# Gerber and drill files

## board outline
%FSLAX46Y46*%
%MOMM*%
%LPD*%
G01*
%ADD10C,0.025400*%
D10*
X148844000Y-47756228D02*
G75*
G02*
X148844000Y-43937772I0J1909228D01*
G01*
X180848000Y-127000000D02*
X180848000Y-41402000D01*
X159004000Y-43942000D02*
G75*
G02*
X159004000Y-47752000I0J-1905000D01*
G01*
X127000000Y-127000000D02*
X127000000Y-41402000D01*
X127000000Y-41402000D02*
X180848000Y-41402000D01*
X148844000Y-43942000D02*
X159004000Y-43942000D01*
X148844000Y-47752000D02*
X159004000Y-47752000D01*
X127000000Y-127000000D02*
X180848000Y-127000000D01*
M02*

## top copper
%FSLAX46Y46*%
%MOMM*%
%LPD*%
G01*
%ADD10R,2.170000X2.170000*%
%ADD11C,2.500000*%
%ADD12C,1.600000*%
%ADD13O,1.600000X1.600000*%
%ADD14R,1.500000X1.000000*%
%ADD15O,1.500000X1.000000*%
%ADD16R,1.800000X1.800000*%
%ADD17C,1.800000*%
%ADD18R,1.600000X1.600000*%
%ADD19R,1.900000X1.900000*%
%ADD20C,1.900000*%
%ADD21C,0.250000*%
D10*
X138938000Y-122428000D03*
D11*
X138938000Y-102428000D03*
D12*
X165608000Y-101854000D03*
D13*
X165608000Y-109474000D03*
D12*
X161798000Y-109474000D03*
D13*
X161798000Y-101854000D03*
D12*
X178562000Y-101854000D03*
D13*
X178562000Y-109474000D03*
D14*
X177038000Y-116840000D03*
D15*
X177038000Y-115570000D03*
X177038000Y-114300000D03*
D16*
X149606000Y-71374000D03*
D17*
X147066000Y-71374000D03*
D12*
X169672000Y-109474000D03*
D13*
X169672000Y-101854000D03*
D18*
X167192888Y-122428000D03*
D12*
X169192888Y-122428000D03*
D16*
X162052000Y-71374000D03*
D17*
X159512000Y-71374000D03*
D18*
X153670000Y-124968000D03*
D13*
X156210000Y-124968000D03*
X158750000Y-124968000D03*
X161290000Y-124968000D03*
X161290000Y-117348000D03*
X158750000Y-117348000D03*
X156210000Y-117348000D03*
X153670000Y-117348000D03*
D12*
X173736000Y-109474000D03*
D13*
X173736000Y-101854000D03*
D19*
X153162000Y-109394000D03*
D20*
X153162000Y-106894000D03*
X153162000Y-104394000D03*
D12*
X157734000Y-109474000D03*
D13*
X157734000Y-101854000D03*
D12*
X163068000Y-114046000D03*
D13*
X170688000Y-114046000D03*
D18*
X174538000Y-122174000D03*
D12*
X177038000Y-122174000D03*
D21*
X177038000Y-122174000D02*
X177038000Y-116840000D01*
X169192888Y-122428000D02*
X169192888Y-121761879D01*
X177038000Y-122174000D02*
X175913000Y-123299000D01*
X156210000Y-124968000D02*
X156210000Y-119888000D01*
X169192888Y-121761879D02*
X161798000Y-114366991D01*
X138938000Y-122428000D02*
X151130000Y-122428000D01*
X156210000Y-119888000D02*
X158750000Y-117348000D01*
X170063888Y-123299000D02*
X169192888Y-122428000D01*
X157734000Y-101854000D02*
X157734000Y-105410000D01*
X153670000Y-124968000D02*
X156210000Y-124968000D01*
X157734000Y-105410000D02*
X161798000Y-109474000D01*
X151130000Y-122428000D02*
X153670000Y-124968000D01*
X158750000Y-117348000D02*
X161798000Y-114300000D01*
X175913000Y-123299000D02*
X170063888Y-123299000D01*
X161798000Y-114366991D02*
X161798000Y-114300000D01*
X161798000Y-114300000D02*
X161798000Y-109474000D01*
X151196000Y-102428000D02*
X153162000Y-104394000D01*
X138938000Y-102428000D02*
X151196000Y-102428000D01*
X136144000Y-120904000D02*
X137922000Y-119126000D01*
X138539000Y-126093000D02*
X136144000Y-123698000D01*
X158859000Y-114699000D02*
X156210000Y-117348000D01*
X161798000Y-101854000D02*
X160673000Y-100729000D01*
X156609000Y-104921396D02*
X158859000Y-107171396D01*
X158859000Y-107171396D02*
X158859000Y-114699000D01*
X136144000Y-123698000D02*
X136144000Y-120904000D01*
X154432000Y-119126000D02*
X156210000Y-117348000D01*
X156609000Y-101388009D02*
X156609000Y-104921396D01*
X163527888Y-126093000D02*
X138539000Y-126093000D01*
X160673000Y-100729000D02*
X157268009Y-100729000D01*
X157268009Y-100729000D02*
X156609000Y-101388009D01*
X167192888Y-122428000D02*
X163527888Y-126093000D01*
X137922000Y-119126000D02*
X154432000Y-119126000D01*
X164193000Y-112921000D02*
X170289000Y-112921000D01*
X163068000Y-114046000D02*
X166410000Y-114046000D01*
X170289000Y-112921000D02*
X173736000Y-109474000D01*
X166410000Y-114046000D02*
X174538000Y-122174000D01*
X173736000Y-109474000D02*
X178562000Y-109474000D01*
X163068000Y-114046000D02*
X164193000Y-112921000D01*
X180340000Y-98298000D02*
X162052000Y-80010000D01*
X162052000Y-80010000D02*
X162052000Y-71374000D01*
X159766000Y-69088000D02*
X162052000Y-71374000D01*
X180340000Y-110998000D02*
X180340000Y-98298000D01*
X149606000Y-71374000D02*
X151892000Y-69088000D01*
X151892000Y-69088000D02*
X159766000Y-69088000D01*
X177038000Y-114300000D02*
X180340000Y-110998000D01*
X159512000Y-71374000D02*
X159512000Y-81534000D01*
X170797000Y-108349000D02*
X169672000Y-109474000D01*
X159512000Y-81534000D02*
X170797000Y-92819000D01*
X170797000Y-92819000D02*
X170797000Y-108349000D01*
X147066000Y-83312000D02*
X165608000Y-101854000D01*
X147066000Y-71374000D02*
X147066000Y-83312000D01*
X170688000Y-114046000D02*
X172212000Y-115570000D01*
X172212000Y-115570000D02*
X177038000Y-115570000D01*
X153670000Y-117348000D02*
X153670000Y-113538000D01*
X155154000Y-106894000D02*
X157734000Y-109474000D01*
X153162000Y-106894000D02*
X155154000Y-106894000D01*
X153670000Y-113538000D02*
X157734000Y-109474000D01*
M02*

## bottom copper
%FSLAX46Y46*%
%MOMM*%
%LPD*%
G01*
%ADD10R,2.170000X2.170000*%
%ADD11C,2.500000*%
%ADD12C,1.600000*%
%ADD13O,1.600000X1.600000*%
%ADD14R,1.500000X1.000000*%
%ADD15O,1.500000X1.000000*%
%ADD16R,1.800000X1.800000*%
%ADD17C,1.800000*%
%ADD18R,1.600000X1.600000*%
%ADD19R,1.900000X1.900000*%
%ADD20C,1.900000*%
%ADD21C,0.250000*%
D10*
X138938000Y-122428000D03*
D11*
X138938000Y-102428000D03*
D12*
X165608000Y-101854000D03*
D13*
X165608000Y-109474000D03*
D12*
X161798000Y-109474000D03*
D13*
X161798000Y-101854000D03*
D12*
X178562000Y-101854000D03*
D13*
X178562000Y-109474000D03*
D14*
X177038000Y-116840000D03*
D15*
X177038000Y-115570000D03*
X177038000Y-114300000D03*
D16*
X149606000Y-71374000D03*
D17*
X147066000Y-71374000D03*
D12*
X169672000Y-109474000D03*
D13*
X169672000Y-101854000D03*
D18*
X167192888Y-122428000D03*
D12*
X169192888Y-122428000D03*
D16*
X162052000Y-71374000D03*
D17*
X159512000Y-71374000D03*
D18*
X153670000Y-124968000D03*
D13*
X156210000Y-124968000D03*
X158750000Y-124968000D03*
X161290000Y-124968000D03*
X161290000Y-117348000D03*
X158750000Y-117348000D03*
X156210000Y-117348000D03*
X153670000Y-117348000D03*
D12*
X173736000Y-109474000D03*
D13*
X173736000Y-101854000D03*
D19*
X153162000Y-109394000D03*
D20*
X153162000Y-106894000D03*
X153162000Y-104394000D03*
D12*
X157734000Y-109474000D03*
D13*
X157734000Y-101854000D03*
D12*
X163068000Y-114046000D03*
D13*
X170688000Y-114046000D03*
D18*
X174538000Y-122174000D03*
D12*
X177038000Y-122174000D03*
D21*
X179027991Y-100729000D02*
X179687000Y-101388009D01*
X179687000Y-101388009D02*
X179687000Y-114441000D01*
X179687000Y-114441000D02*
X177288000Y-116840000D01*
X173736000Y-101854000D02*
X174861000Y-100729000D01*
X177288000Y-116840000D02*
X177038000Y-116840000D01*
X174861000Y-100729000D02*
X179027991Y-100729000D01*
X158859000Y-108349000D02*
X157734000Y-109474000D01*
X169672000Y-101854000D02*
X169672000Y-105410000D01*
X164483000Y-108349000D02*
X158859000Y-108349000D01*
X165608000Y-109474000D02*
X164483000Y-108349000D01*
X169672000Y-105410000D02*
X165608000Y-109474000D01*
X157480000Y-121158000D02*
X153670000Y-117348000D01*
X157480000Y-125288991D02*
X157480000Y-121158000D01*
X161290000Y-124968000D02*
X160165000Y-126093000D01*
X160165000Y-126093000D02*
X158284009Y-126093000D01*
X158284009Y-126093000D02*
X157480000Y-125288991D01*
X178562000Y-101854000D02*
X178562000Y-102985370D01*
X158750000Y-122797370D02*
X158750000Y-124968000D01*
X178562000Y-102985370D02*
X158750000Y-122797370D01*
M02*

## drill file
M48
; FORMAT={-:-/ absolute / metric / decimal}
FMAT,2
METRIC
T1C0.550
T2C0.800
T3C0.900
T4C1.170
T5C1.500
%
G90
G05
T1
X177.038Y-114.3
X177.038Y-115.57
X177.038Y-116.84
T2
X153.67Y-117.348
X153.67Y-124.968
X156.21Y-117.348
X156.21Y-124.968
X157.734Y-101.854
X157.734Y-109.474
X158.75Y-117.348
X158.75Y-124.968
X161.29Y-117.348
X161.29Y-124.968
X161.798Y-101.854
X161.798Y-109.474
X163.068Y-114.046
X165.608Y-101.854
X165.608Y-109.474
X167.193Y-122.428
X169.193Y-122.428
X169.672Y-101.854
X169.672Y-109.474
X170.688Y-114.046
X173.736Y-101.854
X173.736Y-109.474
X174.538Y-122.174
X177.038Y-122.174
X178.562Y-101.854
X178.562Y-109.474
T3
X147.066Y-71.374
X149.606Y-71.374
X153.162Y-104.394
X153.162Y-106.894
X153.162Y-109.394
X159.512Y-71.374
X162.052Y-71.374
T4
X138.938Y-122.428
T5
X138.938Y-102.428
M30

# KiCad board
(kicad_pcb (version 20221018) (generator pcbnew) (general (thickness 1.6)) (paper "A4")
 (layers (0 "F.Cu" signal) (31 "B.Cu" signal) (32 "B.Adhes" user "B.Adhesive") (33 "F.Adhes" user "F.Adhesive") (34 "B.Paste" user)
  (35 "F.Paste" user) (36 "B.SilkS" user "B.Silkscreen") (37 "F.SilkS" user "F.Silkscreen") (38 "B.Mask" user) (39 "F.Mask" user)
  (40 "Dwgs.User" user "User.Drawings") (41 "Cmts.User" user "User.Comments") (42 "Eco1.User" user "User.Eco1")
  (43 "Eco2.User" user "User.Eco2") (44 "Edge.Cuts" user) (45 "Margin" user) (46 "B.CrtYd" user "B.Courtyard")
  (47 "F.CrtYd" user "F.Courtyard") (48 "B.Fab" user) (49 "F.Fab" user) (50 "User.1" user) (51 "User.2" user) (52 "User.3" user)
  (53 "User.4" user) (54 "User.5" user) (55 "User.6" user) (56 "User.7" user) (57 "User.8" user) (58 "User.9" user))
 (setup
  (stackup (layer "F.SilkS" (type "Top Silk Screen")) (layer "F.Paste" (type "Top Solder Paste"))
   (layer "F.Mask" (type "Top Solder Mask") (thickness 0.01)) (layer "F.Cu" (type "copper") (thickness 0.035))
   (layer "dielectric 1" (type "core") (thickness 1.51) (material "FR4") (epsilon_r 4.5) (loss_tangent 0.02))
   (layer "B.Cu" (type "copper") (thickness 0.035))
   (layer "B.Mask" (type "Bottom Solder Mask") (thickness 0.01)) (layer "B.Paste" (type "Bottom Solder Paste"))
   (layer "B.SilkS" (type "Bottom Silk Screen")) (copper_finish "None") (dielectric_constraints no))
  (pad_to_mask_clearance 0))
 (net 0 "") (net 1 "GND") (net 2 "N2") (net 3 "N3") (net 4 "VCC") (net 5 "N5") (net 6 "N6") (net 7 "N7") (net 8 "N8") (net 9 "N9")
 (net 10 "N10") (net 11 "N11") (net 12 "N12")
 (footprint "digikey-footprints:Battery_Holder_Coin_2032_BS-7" (layer "F.Cu") (at 138.938 122.428 90)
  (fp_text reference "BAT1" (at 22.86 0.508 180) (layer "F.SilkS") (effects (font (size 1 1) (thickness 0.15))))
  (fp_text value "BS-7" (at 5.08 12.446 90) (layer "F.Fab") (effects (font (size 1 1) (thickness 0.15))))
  (pad "Neg" thru_hole rect (at 0 0 90) (size 2.17 2.17) (drill 1.17) (layers "*.Cu" "*.Mask") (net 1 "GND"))
  (pad "Pos" thru_hole circle (at 20 0 90) (size 2.5 2.5) (drill 1.5) (layers "*.Cu" "*.Mask") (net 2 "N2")))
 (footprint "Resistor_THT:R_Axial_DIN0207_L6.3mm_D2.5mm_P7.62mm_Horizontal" (layer "F.Cu") (at 165.608 101.854 -90)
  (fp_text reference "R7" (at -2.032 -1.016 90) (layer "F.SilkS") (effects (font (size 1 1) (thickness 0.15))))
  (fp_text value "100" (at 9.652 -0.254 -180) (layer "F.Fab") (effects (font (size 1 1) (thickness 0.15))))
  (pad "1" thru_hole circle (at 0 0 270) (size 1.6 1.6) (drill 0.8) (layers "*.Cu" "*.Mask") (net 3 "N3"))
  (pad "2" thru_hole oval (at 7.62 0 270) (size 1.6 1.6) (drill 0.8) (layers "*.Cu" "*.Mask") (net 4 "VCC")))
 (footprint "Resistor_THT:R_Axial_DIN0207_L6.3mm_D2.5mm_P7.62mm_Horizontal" (layer "F.Cu") (at 161.798 109.474 90)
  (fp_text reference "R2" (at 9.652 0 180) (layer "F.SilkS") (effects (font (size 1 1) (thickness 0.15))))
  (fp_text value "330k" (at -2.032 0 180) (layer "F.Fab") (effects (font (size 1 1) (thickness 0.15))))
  (pad "1" thru_hole circle (at 0 0 90) (size 1.6 1.6) (drill 0.8) (layers "*.Cu" "*.Mask") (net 1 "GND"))
  (pad "2" thru_hole oval (at 7.62 0 90) (size 1.6 1.6) (drill 0.8) (layers "*.Cu" "*.Mask") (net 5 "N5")))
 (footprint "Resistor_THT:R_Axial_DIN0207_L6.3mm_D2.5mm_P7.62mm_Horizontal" (layer "F.Cu") (at 178.562 101.854 -90)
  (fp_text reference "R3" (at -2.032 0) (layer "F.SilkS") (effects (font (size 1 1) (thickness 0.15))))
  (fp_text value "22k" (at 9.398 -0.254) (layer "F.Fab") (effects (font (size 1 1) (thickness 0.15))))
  (pad "1" thru_hole circle (at 0 0 270) (size 1.6 1.6) (drill 0.8) (layers "*.Cu" "*.Mask") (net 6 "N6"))
  (pad "2" thru_hole oval (at 7.62 0 270) (size 1.6 1.6) (drill 0.8) (layers "*.Cu" "*.Mask") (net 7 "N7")))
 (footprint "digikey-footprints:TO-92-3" (layer "F.Cu") (at 177.038 116.84 90)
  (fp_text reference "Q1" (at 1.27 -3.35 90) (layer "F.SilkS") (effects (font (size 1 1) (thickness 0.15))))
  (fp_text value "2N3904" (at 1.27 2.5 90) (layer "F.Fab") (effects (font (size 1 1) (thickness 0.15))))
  (pad "1" thru_hole rect (at 0 0 270) (size 1 1.5) (drill 0.55) (layers "*.Cu" "*.Mask") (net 1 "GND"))
  (pad "2" thru_hole oval (at 1.27 0 270) (size 1 1.5) (drill 0.55) (layers "*.Cu" "*.Mask") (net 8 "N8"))
  (pad "3" thru_hole oval (at 2.54 0 270) (size 1 1.5) (drill 0.55) (layers "*.Cu" "*.Mask") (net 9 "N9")))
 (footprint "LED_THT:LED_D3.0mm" (layer "F.Cu") (at 149.606 71.374 180)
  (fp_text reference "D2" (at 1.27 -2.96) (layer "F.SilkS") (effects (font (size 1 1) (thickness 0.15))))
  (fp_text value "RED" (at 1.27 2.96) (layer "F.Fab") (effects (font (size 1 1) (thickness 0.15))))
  (pad "1" thru_hole rect (at 0 0 180) (size 1.8 1.8) (drill 0.9) (layers "*.Cu" "*.Mask") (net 9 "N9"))
  (pad "2" thru_hole circle (at 2.54 0 180) (size 1.8 1.8) (drill 0.9) (layers "*.Cu" "*.Mask") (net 3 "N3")))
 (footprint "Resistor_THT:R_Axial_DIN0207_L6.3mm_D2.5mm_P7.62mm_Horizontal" (layer "F.Cu") (at 169.672 109.474 90)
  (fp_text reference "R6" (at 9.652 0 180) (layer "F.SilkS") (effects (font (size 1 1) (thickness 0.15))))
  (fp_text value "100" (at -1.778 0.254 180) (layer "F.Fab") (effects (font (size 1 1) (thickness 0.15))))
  (pad "1" thru_hole circle (at 0 0 90) (size 1.6 1.6) (drill 0.8) (layers "*.Cu" "*.Mask") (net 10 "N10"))
  (pad "2" thru_hole oval (at 7.62 0 90) (size 1.6 1.6) (drill 0.8) (layers "*.Cu" "*.Mask") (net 4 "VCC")))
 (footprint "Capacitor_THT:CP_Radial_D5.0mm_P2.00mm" (layer "F.Cu") (at 167.192888 122.428)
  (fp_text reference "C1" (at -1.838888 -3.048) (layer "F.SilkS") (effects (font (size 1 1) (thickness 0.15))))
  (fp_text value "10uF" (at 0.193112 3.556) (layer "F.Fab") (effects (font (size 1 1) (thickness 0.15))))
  (pad "1" thru_hole rect (at 0 0) (size 1.6 1.6) (drill 0.8) (layers "*.Cu" "*.Mask") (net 5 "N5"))
  (pad "2" thru_hole circle (at 2 0) (size 1.6 1.6) (drill 0.8) (layers "*.Cu" "*.Mask") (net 1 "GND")))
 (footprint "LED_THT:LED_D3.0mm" (layer "F.Cu") (at 162.052 71.374 180)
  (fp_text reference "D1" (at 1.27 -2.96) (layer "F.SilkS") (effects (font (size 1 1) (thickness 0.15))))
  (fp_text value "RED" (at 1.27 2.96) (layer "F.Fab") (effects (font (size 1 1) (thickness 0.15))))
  (pad "1" thru_hole rect (at 0 0 180) (size 1.8 1.8) (drill 0.9) (layers "*.Cu" "*.Mask") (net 9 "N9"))
  (pad "2" thru_hole circle (at 2.54 0 180) (size 1.8 1.8) (drill 0.9) (layers "*.Cu" "*.Mask") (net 10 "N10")))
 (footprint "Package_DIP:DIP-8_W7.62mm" (layer "F.Cu") (at 153.67 124.968 90)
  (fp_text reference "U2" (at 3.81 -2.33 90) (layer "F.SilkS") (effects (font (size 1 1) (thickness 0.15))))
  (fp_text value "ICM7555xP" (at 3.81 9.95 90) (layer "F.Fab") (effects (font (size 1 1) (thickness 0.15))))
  (pad "1" thru_hole rect (at 0 0 90) (size 1.6 1.6) (drill 0.8) (layers "*.Cu" "*.Mask") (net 1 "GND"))
  (pad "2" thru_hole oval (at 0 2.54 90) (size 1.6 1.6) (drill 0.8) (layers "*.Cu" "*.Mask") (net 1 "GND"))
  (pad "3" thru_hole oval (at 0 5.08 90) (size 1.6 1.6) (drill 0.8) (layers "*.Cu" "*.Mask") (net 6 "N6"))
  (pad "4" thru_hole oval (at 0 7.62 90) (size 1.6 1.6) (drill 0.8) (layers "*.Cu" "*.Mask") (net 4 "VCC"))
  (pad "5" thru_hole oval (at 7.62 7.62 90) (size 1.6 1.6) (drill 0.8) (layers "*.Cu" "*.Mask") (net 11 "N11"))
  (pad "6" thru_hole oval (at 7.62 5.08 90) (size 1.6 1.6) (drill 0.8) (layers "*.Cu" "*.Mask") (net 1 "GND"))
  (pad "7" thru_hole oval (at 7.62 2.54 90) (size 1.6 1.6) (drill 0.8) (layers "*.Cu" "*.Mask") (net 5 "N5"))
  (pad "8" thru_hole oval (at 7.62 0 90) (size 1.6 1.6) (drill 0.8) (layers "*.Cu" "*.Mask") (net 4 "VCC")))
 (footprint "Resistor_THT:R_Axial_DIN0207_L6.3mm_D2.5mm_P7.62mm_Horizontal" (layer "F.Cu") (at 173.736 109.474 90)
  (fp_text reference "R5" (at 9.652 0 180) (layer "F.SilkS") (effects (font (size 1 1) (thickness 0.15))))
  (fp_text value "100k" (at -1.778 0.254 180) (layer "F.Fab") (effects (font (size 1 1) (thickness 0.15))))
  (pad "1" thru_hole circle (at 0 0 90) (size 1.6 1.6) (drill 0.8) (layers "*.Cu" "*.Mask") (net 7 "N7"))
  (pad "2" thru_hole oval (at 7.62 0 90) (size 1.6 1.6) (drill 0.8) (layers "*.Cu" "*.Mask") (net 1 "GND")))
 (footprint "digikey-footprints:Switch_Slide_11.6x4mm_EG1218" (layer "F.Cu") (at 153.162 109.394 90)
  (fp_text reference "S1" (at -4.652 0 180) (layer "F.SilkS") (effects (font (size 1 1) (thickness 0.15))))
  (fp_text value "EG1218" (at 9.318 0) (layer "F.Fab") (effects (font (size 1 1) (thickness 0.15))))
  (pad "1" thru_hole rect (at 0 0 90) (size 1.9 1.9) (drill 0.9) (layers "*.Cu" "*.Mask") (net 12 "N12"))
  (pad "2" thru_hole circle (at 2.5 0 90) (size 1.9 1.9) (drill 0.9) (layers "*.Cu" "*.Mask") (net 4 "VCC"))
  (pad "3" thru_hole circle (at 5 0 90) (size 1.9 1.9) (drill 0.9) (layers "*.Cu" "*.Mask") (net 2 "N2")))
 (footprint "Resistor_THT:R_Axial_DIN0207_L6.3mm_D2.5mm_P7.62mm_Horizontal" (layer "F.Cu") (at 157.734 109.474 90)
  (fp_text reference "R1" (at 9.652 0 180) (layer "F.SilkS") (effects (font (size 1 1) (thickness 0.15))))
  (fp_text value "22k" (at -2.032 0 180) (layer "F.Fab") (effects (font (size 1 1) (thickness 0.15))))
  (pad "1" thru_hole circle (at 0 0 90) (size 1.6 1.6) (drill 0.8) (layers "*.Cu" "*.Mask") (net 4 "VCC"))
  (pad "2" thru_hole oval (at 7.62 0 90) (size 1.6 1.6) (drill 0.8) (layers "*.Cu" "*.Mask") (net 1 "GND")))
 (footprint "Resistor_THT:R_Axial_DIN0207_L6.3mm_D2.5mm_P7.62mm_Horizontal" (layer "F.Cu") (at 163.068 114.046)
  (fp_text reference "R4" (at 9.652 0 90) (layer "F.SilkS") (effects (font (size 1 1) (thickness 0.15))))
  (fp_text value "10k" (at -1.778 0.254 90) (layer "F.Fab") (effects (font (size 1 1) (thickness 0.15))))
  (pad "1" thru_hole circle (at 0 0) (size 1.6 1.6) (drill 0.8) (layers "*.Cu" "*.Mask") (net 7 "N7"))
  (pad "2" thru_hole oval (at 7.62 0) (size 1.6 1.6) (drill 0.8) (layers "*.Cu" "*.Mask") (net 8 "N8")))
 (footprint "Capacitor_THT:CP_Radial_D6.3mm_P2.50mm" (layer "F.Cu") (at 174.538 122.174)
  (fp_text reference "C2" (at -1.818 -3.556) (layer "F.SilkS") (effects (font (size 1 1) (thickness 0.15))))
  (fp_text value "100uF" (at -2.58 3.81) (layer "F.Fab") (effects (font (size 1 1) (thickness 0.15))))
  (pad "1" thru_hole rect (at 0 0) (size 1.6 1.6) (drill 0.8) (layers "*.Cu" "*.Mask") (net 7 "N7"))
  (pad "2" thru_hole circle (at 2.5 0) (size 1.6 1.6) (drill 0.8) (layers "*.Cu" "*.Mask") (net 1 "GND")))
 (gr_arc (start 148.844 47.756228) (mid 146.934772 45.847) (end 148.844 43.937772) (stroke (width 0.0254) (type default))
  (layer "Edge.Cuts"))
 (gr_line (start 180.848 127) (end 180.848 41.402) (stroke (width 0.0254) (type default)) (layer "Edge.Cuts"))
 (gr_arc (start 159.004 43.942) (mid 160.909 45.847) (end 159.004 47.752) (stroke (width 0.0254) (type default)) (layer "Edge.Cuts"))
 (gr_line (start 127 127) (end 127 41.402) (stroke (width 0.0254) (type default)) (layer "Edge.Cuts"))
 (gr_line (start 127 41.402) (end 180.848 41.402) (stroke (width 0.0254) (type default)) (layer "Edge.Cuts"))
 (gr_line (start 148.844 43.942) (end 159.004 43.942) (stroke (width 0.0254) (type default)) (layer "Edge.Cuts"))
 (gr_line (start 148.844 47.752) (end 159.004 47.752) (stroke (width 0.0254) (type default)) (layer "Edge.Cuts"))
 (gr_line (start 127 127) (end 180.848 127) (stroke (width 0.0254) (type default)) (layer "Edge.Cuts"))
 (segment (start 177.038 122.174) (end 177.038 116.84) (width 0.25) (layer "F.Cu") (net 1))
 (segment (start 169.192888 122.428) (end 169.192888 121.761879) (width 0.25) (layer "F.Cu") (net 1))
 (segment (start 177.038 122.174) (end 175.913 123.299) (width 0.25) (layer "F.Cu") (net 1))
 (segment (start 156.21 124.968) (end 156.21 119.888) (width 0.25) (layer "F.Cu") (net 1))
 (segment (start 169.192888 121.761879) (end 161.798 114.366991) (width 0.25) (layer "F.Cu") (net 1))
 (segment (start 138.938 122.428) (end 151.13 122.428) (width 0.25) (layer "F.Cu") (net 1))
 (segment (start 156.21 119.888) (end 158.75 117.348) (width 0.25) (layer "F.Cu") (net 1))
 (segment (start 170.063888 123.299) (end 169.192888 122.428) (width 0.25) (layer "F.Cu") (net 1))
 (segment (start 157.734 101.854) (end 157.734 105.41) (width 0.25) (layer "F.Cu") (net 1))
 (segment (start 153.67 124.968) (end 156.21 124.968) (width 0.25) (layer "F.Cu") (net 1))
 (segment (start 157.734 105.41) (end 161.798 109.474) (width 0.25) (layer "F.Cu") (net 1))
 (segment (start 151.13 122.428) (end 153.67 124.968) (width 0.25) (layer "F.Cu") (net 1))
 (segment (start 158.75 117.348) (end 161.798 114.3) (width 0.25) (layer "F.Cu") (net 1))
 (segment (start 175.913 123.299) (end 170.063888 123.299) (width 0.25) (layer "F.Cu") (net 1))
 (segment (start 161.798 114.366991) (end 161.798 114.3) (width 0.25) (layer "F.Cu") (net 1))
 (segment (start 161.798 114.3) (end 161.798 109.474) (width 0.25) (layer "F.Cu") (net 1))
 (segment (start 179.027991 100.729) (end 179.687 101.388009) (width 0.25) (layer "B.Cu") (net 1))
 (segment (start 179.687 101.388009) (end 179.687 114.441) (width 0.25) (layer "B.Cu") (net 1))
 (segment (start 179.687 114.441) (end 177.288 116.84) (width 0.25) (layer "B.Cu") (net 1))
 (segment (start 173.736 101.854) (end 174.861 100.729) (width 0.25) (layer "B.Cu") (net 1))
 (segment (start 177.288 116.84) (end 177.038 116.84) (width 0.25) (layer "B.Cu") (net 1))
 (segment (start 174.861 100.729) (end 179.027991 100.729) (width 0.25) (layer "B.Cu") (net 1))
 (segment (start 151.196 102.428) (end 153.162 104.394) (width 0.25) (layer "F.Cu") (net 2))
 (segment (start 138.938 102.428) (end 151.196 102.428) (width 0.25) (layer "F.Cu") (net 2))
 (segment (start 136.144 120.904) (end 137.922 119.126) (width 0.25) (layer "F.Cu") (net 5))
 (segment (start 138.539 126.093) (end 136.144 123.698) (width 0.25) (layer "F.Cu") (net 5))
 (segment (start 158.859 114.699) (end 156.21 117.348) (width 0.25) (layer "F.Cu") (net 5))
 (segment (start 161.798 101.854) (end 160.673 100.729) (width 0.25) (layer "F.Cu") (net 5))
 (segment (start 156.609 104.921396) (end 158.859 107.171396) (width 0.25) (layer "F.Cu") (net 5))
 (segment (start 158.859 107.171396) (end 158.859 114.699) (width 0.25) (layer "F.Cu") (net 5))
 (segment (start 136.144 123.698) (end 136.144 120.904) (width 0.25) (layer "F.Cu") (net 5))
 (segment (start 154.432 119.126) (end 156.21 117.348) (width 0.25) (layer "F.Cu") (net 5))
 (segment (start 156.609 101.388009) (end 156.609 104.921396) (width 0.25) (layer "F.Cu") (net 5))
 (segment (start 163.527888 126.093) (end 138.539 126.093) (width 0.25) (layer "F.Cu") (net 5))
 (segment (start 160.673 100.729) (end 157.268009 100.729) (width 0.25) (layer "F.Cu") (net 5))
 (segment (start 157.268009 100.729) (end 156.609 101.388009) (width 0.25) (layer "F.Cu") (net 5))
 (segment (start 167.192888 122.428) (end 163.527888 126.093) (width 0.25) (layer "F.Cu") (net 5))
 (segment (start 137.922 119.126) (end 154.432 119.126) (width 0.25) (layer "F.Cu") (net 5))
 (segment (start 164.193 112.921) (end 170.289 112.921) (width 0.25) (layer "F.Cu") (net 7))
 (segment (start 163.068 114.046) (end 166.41 114.046) (width 0.25) (layer "F.Cu") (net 7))
 (segment (start 170.289 112.921) (end 173.736 109.474) (width 0.25) (layer "F.Cu") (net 7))
 (segment (start 166.41 114.046) (end 174.538 122.174) (width 0.25) (layer "F.Cu") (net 7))
 (segment (start 173.736 109.474) (end 178.562 109.474) (width 0.25) (layer "F.Cu") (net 7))
 (segment (start 163.068 114.046) (end 164.193 112.921) (width 0.25) (layer "F.Cu") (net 7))
 (segment (start 180.34 98.298) (end 162.052 80.01) (width 0.25) (layer "F.Cu") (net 9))
 (segment (start 162.052 80.01) (end 162.052 71.374) (width 0.25) (layer "F.Cu") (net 9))
 (segment (start 159.766 69.088) (end 162.052 71.374) (width 0.25) (layer "F.Cu") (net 9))
 (segment (start 180.34 110.998) (end 180.34 98.298) (width 0.25) (layer "F.Cu") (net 9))
 (segment (start 149.606 71.374) (end 151.892 69.088) (width 0.25) (layer "F.Cu") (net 9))
 (segment (start 151.892 69.088) (end 159.766 69.088) (width 0.25) (layer "F.Cu") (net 9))
 (segment (start 177.038 114.3) (end 180.34 110.998) (width 0.25) (layer "F.Cu") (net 9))
 (segment (start 159.512 71.374) (end 159.512 81.534) (width 0.25) (layer "F.Cu") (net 10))
 (segment (start 170.797 108.349) (end 169.672 109.474) (width 0.25) (layer "F.Cu") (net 10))
 (segment (start 159.512 81.534) (end 170.797 92.819) (width 0.25) (layer "F.Cu") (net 10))
 (segment (start 170.797 92.819) (end 170.797 108.349) (width 0.25) (layer "F.Cu") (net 10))
 (segment (start 147.066 83.312) (end 165.608 101.854) (width 0.25) (layer "F.Cu") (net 3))
 (segment (start 147.066 71.374) (end 147.066 83.312) (width 0.25) (layer "F.Cu") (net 3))
 (segment (start 170.688 114.046) (end 172.212 115.57) (width 0.25) (layer "F.Cu") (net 8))
 (segment (start 172.212 115.57) (end 177.038 115.57) (width 0.25) (layer "F.Cu") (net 8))
 (segment (start 153.67 117.348) (end 153.67 113.538) (width 0.25) (layer "F.Cu") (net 4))
 (segment (start 155.154 106.894) (end 157.734 109.474) (width 0.25) (layer "F.Cu") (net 4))
 (segment (start 153.162 106.894) (end 155.154 106.894) (width 0.25) (layer "F.Cu") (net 4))
 (segment (start 153.67 113.538) (end 157.734 109.474) (width 0.25) (layer "F.Cu") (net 4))
 (segment (start 158.859 108.349) (end 157.734 109.474) (width 0.25) (layer "B.Cu") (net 4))
 (segment (start 169.672 101.854) (end 169.672 105.41) (width 0.25) (layer "B.Cu") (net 4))
 (segment (start 164.483 108.349) (end 158.859 108.349) (width 0.25) (layer "B.Cu") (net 4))
 (segment (start 165.608 109.474) (end 164.483 108.349) (width 0.25) (layer "B.Cu") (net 4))
 (segment (start 169.672 105.41) (end 165.608 109.474) (width 0.25) (layer "B.Cu") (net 4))
 (segment (start 157.48 121.158) (end 153.67 117.348) (width 0.25) (layer "B.Cu") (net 4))
 (segment (start 157.48 125.288991) (end 157.48 121.158) (width 0.25) (layer "B.Cu") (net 4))
 (segment (start 161.29 124.968) (end 160.165 126.093) (width 0.25) (layer "B.Cu") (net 4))
 (segment (start 160.165 126.093) (end 158.284009 126.093) (width 0.25) (layer "B.Cu") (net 4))
 (segment (start 158.284009 126.093) (end 157.48 125.288991) (width 0.25) (layer "B.Cu") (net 4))
 (segment (start 178.562 101.854) (end 178.562 102.98537) (width 0.25) (layer "B.Cu") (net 6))
 (segment (start 158.75 122.79737) (end 158.75 124.968) (width 0.25) (layer "B.Cu") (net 6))
 (segment (start 178.562 102.98537) (end 158.75 122.79737) (width 0.25) (layer "B.Cu") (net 6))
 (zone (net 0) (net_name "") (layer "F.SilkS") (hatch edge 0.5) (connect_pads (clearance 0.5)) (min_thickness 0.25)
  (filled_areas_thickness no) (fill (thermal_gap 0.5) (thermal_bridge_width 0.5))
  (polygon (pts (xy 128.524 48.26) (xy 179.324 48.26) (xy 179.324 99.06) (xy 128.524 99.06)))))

